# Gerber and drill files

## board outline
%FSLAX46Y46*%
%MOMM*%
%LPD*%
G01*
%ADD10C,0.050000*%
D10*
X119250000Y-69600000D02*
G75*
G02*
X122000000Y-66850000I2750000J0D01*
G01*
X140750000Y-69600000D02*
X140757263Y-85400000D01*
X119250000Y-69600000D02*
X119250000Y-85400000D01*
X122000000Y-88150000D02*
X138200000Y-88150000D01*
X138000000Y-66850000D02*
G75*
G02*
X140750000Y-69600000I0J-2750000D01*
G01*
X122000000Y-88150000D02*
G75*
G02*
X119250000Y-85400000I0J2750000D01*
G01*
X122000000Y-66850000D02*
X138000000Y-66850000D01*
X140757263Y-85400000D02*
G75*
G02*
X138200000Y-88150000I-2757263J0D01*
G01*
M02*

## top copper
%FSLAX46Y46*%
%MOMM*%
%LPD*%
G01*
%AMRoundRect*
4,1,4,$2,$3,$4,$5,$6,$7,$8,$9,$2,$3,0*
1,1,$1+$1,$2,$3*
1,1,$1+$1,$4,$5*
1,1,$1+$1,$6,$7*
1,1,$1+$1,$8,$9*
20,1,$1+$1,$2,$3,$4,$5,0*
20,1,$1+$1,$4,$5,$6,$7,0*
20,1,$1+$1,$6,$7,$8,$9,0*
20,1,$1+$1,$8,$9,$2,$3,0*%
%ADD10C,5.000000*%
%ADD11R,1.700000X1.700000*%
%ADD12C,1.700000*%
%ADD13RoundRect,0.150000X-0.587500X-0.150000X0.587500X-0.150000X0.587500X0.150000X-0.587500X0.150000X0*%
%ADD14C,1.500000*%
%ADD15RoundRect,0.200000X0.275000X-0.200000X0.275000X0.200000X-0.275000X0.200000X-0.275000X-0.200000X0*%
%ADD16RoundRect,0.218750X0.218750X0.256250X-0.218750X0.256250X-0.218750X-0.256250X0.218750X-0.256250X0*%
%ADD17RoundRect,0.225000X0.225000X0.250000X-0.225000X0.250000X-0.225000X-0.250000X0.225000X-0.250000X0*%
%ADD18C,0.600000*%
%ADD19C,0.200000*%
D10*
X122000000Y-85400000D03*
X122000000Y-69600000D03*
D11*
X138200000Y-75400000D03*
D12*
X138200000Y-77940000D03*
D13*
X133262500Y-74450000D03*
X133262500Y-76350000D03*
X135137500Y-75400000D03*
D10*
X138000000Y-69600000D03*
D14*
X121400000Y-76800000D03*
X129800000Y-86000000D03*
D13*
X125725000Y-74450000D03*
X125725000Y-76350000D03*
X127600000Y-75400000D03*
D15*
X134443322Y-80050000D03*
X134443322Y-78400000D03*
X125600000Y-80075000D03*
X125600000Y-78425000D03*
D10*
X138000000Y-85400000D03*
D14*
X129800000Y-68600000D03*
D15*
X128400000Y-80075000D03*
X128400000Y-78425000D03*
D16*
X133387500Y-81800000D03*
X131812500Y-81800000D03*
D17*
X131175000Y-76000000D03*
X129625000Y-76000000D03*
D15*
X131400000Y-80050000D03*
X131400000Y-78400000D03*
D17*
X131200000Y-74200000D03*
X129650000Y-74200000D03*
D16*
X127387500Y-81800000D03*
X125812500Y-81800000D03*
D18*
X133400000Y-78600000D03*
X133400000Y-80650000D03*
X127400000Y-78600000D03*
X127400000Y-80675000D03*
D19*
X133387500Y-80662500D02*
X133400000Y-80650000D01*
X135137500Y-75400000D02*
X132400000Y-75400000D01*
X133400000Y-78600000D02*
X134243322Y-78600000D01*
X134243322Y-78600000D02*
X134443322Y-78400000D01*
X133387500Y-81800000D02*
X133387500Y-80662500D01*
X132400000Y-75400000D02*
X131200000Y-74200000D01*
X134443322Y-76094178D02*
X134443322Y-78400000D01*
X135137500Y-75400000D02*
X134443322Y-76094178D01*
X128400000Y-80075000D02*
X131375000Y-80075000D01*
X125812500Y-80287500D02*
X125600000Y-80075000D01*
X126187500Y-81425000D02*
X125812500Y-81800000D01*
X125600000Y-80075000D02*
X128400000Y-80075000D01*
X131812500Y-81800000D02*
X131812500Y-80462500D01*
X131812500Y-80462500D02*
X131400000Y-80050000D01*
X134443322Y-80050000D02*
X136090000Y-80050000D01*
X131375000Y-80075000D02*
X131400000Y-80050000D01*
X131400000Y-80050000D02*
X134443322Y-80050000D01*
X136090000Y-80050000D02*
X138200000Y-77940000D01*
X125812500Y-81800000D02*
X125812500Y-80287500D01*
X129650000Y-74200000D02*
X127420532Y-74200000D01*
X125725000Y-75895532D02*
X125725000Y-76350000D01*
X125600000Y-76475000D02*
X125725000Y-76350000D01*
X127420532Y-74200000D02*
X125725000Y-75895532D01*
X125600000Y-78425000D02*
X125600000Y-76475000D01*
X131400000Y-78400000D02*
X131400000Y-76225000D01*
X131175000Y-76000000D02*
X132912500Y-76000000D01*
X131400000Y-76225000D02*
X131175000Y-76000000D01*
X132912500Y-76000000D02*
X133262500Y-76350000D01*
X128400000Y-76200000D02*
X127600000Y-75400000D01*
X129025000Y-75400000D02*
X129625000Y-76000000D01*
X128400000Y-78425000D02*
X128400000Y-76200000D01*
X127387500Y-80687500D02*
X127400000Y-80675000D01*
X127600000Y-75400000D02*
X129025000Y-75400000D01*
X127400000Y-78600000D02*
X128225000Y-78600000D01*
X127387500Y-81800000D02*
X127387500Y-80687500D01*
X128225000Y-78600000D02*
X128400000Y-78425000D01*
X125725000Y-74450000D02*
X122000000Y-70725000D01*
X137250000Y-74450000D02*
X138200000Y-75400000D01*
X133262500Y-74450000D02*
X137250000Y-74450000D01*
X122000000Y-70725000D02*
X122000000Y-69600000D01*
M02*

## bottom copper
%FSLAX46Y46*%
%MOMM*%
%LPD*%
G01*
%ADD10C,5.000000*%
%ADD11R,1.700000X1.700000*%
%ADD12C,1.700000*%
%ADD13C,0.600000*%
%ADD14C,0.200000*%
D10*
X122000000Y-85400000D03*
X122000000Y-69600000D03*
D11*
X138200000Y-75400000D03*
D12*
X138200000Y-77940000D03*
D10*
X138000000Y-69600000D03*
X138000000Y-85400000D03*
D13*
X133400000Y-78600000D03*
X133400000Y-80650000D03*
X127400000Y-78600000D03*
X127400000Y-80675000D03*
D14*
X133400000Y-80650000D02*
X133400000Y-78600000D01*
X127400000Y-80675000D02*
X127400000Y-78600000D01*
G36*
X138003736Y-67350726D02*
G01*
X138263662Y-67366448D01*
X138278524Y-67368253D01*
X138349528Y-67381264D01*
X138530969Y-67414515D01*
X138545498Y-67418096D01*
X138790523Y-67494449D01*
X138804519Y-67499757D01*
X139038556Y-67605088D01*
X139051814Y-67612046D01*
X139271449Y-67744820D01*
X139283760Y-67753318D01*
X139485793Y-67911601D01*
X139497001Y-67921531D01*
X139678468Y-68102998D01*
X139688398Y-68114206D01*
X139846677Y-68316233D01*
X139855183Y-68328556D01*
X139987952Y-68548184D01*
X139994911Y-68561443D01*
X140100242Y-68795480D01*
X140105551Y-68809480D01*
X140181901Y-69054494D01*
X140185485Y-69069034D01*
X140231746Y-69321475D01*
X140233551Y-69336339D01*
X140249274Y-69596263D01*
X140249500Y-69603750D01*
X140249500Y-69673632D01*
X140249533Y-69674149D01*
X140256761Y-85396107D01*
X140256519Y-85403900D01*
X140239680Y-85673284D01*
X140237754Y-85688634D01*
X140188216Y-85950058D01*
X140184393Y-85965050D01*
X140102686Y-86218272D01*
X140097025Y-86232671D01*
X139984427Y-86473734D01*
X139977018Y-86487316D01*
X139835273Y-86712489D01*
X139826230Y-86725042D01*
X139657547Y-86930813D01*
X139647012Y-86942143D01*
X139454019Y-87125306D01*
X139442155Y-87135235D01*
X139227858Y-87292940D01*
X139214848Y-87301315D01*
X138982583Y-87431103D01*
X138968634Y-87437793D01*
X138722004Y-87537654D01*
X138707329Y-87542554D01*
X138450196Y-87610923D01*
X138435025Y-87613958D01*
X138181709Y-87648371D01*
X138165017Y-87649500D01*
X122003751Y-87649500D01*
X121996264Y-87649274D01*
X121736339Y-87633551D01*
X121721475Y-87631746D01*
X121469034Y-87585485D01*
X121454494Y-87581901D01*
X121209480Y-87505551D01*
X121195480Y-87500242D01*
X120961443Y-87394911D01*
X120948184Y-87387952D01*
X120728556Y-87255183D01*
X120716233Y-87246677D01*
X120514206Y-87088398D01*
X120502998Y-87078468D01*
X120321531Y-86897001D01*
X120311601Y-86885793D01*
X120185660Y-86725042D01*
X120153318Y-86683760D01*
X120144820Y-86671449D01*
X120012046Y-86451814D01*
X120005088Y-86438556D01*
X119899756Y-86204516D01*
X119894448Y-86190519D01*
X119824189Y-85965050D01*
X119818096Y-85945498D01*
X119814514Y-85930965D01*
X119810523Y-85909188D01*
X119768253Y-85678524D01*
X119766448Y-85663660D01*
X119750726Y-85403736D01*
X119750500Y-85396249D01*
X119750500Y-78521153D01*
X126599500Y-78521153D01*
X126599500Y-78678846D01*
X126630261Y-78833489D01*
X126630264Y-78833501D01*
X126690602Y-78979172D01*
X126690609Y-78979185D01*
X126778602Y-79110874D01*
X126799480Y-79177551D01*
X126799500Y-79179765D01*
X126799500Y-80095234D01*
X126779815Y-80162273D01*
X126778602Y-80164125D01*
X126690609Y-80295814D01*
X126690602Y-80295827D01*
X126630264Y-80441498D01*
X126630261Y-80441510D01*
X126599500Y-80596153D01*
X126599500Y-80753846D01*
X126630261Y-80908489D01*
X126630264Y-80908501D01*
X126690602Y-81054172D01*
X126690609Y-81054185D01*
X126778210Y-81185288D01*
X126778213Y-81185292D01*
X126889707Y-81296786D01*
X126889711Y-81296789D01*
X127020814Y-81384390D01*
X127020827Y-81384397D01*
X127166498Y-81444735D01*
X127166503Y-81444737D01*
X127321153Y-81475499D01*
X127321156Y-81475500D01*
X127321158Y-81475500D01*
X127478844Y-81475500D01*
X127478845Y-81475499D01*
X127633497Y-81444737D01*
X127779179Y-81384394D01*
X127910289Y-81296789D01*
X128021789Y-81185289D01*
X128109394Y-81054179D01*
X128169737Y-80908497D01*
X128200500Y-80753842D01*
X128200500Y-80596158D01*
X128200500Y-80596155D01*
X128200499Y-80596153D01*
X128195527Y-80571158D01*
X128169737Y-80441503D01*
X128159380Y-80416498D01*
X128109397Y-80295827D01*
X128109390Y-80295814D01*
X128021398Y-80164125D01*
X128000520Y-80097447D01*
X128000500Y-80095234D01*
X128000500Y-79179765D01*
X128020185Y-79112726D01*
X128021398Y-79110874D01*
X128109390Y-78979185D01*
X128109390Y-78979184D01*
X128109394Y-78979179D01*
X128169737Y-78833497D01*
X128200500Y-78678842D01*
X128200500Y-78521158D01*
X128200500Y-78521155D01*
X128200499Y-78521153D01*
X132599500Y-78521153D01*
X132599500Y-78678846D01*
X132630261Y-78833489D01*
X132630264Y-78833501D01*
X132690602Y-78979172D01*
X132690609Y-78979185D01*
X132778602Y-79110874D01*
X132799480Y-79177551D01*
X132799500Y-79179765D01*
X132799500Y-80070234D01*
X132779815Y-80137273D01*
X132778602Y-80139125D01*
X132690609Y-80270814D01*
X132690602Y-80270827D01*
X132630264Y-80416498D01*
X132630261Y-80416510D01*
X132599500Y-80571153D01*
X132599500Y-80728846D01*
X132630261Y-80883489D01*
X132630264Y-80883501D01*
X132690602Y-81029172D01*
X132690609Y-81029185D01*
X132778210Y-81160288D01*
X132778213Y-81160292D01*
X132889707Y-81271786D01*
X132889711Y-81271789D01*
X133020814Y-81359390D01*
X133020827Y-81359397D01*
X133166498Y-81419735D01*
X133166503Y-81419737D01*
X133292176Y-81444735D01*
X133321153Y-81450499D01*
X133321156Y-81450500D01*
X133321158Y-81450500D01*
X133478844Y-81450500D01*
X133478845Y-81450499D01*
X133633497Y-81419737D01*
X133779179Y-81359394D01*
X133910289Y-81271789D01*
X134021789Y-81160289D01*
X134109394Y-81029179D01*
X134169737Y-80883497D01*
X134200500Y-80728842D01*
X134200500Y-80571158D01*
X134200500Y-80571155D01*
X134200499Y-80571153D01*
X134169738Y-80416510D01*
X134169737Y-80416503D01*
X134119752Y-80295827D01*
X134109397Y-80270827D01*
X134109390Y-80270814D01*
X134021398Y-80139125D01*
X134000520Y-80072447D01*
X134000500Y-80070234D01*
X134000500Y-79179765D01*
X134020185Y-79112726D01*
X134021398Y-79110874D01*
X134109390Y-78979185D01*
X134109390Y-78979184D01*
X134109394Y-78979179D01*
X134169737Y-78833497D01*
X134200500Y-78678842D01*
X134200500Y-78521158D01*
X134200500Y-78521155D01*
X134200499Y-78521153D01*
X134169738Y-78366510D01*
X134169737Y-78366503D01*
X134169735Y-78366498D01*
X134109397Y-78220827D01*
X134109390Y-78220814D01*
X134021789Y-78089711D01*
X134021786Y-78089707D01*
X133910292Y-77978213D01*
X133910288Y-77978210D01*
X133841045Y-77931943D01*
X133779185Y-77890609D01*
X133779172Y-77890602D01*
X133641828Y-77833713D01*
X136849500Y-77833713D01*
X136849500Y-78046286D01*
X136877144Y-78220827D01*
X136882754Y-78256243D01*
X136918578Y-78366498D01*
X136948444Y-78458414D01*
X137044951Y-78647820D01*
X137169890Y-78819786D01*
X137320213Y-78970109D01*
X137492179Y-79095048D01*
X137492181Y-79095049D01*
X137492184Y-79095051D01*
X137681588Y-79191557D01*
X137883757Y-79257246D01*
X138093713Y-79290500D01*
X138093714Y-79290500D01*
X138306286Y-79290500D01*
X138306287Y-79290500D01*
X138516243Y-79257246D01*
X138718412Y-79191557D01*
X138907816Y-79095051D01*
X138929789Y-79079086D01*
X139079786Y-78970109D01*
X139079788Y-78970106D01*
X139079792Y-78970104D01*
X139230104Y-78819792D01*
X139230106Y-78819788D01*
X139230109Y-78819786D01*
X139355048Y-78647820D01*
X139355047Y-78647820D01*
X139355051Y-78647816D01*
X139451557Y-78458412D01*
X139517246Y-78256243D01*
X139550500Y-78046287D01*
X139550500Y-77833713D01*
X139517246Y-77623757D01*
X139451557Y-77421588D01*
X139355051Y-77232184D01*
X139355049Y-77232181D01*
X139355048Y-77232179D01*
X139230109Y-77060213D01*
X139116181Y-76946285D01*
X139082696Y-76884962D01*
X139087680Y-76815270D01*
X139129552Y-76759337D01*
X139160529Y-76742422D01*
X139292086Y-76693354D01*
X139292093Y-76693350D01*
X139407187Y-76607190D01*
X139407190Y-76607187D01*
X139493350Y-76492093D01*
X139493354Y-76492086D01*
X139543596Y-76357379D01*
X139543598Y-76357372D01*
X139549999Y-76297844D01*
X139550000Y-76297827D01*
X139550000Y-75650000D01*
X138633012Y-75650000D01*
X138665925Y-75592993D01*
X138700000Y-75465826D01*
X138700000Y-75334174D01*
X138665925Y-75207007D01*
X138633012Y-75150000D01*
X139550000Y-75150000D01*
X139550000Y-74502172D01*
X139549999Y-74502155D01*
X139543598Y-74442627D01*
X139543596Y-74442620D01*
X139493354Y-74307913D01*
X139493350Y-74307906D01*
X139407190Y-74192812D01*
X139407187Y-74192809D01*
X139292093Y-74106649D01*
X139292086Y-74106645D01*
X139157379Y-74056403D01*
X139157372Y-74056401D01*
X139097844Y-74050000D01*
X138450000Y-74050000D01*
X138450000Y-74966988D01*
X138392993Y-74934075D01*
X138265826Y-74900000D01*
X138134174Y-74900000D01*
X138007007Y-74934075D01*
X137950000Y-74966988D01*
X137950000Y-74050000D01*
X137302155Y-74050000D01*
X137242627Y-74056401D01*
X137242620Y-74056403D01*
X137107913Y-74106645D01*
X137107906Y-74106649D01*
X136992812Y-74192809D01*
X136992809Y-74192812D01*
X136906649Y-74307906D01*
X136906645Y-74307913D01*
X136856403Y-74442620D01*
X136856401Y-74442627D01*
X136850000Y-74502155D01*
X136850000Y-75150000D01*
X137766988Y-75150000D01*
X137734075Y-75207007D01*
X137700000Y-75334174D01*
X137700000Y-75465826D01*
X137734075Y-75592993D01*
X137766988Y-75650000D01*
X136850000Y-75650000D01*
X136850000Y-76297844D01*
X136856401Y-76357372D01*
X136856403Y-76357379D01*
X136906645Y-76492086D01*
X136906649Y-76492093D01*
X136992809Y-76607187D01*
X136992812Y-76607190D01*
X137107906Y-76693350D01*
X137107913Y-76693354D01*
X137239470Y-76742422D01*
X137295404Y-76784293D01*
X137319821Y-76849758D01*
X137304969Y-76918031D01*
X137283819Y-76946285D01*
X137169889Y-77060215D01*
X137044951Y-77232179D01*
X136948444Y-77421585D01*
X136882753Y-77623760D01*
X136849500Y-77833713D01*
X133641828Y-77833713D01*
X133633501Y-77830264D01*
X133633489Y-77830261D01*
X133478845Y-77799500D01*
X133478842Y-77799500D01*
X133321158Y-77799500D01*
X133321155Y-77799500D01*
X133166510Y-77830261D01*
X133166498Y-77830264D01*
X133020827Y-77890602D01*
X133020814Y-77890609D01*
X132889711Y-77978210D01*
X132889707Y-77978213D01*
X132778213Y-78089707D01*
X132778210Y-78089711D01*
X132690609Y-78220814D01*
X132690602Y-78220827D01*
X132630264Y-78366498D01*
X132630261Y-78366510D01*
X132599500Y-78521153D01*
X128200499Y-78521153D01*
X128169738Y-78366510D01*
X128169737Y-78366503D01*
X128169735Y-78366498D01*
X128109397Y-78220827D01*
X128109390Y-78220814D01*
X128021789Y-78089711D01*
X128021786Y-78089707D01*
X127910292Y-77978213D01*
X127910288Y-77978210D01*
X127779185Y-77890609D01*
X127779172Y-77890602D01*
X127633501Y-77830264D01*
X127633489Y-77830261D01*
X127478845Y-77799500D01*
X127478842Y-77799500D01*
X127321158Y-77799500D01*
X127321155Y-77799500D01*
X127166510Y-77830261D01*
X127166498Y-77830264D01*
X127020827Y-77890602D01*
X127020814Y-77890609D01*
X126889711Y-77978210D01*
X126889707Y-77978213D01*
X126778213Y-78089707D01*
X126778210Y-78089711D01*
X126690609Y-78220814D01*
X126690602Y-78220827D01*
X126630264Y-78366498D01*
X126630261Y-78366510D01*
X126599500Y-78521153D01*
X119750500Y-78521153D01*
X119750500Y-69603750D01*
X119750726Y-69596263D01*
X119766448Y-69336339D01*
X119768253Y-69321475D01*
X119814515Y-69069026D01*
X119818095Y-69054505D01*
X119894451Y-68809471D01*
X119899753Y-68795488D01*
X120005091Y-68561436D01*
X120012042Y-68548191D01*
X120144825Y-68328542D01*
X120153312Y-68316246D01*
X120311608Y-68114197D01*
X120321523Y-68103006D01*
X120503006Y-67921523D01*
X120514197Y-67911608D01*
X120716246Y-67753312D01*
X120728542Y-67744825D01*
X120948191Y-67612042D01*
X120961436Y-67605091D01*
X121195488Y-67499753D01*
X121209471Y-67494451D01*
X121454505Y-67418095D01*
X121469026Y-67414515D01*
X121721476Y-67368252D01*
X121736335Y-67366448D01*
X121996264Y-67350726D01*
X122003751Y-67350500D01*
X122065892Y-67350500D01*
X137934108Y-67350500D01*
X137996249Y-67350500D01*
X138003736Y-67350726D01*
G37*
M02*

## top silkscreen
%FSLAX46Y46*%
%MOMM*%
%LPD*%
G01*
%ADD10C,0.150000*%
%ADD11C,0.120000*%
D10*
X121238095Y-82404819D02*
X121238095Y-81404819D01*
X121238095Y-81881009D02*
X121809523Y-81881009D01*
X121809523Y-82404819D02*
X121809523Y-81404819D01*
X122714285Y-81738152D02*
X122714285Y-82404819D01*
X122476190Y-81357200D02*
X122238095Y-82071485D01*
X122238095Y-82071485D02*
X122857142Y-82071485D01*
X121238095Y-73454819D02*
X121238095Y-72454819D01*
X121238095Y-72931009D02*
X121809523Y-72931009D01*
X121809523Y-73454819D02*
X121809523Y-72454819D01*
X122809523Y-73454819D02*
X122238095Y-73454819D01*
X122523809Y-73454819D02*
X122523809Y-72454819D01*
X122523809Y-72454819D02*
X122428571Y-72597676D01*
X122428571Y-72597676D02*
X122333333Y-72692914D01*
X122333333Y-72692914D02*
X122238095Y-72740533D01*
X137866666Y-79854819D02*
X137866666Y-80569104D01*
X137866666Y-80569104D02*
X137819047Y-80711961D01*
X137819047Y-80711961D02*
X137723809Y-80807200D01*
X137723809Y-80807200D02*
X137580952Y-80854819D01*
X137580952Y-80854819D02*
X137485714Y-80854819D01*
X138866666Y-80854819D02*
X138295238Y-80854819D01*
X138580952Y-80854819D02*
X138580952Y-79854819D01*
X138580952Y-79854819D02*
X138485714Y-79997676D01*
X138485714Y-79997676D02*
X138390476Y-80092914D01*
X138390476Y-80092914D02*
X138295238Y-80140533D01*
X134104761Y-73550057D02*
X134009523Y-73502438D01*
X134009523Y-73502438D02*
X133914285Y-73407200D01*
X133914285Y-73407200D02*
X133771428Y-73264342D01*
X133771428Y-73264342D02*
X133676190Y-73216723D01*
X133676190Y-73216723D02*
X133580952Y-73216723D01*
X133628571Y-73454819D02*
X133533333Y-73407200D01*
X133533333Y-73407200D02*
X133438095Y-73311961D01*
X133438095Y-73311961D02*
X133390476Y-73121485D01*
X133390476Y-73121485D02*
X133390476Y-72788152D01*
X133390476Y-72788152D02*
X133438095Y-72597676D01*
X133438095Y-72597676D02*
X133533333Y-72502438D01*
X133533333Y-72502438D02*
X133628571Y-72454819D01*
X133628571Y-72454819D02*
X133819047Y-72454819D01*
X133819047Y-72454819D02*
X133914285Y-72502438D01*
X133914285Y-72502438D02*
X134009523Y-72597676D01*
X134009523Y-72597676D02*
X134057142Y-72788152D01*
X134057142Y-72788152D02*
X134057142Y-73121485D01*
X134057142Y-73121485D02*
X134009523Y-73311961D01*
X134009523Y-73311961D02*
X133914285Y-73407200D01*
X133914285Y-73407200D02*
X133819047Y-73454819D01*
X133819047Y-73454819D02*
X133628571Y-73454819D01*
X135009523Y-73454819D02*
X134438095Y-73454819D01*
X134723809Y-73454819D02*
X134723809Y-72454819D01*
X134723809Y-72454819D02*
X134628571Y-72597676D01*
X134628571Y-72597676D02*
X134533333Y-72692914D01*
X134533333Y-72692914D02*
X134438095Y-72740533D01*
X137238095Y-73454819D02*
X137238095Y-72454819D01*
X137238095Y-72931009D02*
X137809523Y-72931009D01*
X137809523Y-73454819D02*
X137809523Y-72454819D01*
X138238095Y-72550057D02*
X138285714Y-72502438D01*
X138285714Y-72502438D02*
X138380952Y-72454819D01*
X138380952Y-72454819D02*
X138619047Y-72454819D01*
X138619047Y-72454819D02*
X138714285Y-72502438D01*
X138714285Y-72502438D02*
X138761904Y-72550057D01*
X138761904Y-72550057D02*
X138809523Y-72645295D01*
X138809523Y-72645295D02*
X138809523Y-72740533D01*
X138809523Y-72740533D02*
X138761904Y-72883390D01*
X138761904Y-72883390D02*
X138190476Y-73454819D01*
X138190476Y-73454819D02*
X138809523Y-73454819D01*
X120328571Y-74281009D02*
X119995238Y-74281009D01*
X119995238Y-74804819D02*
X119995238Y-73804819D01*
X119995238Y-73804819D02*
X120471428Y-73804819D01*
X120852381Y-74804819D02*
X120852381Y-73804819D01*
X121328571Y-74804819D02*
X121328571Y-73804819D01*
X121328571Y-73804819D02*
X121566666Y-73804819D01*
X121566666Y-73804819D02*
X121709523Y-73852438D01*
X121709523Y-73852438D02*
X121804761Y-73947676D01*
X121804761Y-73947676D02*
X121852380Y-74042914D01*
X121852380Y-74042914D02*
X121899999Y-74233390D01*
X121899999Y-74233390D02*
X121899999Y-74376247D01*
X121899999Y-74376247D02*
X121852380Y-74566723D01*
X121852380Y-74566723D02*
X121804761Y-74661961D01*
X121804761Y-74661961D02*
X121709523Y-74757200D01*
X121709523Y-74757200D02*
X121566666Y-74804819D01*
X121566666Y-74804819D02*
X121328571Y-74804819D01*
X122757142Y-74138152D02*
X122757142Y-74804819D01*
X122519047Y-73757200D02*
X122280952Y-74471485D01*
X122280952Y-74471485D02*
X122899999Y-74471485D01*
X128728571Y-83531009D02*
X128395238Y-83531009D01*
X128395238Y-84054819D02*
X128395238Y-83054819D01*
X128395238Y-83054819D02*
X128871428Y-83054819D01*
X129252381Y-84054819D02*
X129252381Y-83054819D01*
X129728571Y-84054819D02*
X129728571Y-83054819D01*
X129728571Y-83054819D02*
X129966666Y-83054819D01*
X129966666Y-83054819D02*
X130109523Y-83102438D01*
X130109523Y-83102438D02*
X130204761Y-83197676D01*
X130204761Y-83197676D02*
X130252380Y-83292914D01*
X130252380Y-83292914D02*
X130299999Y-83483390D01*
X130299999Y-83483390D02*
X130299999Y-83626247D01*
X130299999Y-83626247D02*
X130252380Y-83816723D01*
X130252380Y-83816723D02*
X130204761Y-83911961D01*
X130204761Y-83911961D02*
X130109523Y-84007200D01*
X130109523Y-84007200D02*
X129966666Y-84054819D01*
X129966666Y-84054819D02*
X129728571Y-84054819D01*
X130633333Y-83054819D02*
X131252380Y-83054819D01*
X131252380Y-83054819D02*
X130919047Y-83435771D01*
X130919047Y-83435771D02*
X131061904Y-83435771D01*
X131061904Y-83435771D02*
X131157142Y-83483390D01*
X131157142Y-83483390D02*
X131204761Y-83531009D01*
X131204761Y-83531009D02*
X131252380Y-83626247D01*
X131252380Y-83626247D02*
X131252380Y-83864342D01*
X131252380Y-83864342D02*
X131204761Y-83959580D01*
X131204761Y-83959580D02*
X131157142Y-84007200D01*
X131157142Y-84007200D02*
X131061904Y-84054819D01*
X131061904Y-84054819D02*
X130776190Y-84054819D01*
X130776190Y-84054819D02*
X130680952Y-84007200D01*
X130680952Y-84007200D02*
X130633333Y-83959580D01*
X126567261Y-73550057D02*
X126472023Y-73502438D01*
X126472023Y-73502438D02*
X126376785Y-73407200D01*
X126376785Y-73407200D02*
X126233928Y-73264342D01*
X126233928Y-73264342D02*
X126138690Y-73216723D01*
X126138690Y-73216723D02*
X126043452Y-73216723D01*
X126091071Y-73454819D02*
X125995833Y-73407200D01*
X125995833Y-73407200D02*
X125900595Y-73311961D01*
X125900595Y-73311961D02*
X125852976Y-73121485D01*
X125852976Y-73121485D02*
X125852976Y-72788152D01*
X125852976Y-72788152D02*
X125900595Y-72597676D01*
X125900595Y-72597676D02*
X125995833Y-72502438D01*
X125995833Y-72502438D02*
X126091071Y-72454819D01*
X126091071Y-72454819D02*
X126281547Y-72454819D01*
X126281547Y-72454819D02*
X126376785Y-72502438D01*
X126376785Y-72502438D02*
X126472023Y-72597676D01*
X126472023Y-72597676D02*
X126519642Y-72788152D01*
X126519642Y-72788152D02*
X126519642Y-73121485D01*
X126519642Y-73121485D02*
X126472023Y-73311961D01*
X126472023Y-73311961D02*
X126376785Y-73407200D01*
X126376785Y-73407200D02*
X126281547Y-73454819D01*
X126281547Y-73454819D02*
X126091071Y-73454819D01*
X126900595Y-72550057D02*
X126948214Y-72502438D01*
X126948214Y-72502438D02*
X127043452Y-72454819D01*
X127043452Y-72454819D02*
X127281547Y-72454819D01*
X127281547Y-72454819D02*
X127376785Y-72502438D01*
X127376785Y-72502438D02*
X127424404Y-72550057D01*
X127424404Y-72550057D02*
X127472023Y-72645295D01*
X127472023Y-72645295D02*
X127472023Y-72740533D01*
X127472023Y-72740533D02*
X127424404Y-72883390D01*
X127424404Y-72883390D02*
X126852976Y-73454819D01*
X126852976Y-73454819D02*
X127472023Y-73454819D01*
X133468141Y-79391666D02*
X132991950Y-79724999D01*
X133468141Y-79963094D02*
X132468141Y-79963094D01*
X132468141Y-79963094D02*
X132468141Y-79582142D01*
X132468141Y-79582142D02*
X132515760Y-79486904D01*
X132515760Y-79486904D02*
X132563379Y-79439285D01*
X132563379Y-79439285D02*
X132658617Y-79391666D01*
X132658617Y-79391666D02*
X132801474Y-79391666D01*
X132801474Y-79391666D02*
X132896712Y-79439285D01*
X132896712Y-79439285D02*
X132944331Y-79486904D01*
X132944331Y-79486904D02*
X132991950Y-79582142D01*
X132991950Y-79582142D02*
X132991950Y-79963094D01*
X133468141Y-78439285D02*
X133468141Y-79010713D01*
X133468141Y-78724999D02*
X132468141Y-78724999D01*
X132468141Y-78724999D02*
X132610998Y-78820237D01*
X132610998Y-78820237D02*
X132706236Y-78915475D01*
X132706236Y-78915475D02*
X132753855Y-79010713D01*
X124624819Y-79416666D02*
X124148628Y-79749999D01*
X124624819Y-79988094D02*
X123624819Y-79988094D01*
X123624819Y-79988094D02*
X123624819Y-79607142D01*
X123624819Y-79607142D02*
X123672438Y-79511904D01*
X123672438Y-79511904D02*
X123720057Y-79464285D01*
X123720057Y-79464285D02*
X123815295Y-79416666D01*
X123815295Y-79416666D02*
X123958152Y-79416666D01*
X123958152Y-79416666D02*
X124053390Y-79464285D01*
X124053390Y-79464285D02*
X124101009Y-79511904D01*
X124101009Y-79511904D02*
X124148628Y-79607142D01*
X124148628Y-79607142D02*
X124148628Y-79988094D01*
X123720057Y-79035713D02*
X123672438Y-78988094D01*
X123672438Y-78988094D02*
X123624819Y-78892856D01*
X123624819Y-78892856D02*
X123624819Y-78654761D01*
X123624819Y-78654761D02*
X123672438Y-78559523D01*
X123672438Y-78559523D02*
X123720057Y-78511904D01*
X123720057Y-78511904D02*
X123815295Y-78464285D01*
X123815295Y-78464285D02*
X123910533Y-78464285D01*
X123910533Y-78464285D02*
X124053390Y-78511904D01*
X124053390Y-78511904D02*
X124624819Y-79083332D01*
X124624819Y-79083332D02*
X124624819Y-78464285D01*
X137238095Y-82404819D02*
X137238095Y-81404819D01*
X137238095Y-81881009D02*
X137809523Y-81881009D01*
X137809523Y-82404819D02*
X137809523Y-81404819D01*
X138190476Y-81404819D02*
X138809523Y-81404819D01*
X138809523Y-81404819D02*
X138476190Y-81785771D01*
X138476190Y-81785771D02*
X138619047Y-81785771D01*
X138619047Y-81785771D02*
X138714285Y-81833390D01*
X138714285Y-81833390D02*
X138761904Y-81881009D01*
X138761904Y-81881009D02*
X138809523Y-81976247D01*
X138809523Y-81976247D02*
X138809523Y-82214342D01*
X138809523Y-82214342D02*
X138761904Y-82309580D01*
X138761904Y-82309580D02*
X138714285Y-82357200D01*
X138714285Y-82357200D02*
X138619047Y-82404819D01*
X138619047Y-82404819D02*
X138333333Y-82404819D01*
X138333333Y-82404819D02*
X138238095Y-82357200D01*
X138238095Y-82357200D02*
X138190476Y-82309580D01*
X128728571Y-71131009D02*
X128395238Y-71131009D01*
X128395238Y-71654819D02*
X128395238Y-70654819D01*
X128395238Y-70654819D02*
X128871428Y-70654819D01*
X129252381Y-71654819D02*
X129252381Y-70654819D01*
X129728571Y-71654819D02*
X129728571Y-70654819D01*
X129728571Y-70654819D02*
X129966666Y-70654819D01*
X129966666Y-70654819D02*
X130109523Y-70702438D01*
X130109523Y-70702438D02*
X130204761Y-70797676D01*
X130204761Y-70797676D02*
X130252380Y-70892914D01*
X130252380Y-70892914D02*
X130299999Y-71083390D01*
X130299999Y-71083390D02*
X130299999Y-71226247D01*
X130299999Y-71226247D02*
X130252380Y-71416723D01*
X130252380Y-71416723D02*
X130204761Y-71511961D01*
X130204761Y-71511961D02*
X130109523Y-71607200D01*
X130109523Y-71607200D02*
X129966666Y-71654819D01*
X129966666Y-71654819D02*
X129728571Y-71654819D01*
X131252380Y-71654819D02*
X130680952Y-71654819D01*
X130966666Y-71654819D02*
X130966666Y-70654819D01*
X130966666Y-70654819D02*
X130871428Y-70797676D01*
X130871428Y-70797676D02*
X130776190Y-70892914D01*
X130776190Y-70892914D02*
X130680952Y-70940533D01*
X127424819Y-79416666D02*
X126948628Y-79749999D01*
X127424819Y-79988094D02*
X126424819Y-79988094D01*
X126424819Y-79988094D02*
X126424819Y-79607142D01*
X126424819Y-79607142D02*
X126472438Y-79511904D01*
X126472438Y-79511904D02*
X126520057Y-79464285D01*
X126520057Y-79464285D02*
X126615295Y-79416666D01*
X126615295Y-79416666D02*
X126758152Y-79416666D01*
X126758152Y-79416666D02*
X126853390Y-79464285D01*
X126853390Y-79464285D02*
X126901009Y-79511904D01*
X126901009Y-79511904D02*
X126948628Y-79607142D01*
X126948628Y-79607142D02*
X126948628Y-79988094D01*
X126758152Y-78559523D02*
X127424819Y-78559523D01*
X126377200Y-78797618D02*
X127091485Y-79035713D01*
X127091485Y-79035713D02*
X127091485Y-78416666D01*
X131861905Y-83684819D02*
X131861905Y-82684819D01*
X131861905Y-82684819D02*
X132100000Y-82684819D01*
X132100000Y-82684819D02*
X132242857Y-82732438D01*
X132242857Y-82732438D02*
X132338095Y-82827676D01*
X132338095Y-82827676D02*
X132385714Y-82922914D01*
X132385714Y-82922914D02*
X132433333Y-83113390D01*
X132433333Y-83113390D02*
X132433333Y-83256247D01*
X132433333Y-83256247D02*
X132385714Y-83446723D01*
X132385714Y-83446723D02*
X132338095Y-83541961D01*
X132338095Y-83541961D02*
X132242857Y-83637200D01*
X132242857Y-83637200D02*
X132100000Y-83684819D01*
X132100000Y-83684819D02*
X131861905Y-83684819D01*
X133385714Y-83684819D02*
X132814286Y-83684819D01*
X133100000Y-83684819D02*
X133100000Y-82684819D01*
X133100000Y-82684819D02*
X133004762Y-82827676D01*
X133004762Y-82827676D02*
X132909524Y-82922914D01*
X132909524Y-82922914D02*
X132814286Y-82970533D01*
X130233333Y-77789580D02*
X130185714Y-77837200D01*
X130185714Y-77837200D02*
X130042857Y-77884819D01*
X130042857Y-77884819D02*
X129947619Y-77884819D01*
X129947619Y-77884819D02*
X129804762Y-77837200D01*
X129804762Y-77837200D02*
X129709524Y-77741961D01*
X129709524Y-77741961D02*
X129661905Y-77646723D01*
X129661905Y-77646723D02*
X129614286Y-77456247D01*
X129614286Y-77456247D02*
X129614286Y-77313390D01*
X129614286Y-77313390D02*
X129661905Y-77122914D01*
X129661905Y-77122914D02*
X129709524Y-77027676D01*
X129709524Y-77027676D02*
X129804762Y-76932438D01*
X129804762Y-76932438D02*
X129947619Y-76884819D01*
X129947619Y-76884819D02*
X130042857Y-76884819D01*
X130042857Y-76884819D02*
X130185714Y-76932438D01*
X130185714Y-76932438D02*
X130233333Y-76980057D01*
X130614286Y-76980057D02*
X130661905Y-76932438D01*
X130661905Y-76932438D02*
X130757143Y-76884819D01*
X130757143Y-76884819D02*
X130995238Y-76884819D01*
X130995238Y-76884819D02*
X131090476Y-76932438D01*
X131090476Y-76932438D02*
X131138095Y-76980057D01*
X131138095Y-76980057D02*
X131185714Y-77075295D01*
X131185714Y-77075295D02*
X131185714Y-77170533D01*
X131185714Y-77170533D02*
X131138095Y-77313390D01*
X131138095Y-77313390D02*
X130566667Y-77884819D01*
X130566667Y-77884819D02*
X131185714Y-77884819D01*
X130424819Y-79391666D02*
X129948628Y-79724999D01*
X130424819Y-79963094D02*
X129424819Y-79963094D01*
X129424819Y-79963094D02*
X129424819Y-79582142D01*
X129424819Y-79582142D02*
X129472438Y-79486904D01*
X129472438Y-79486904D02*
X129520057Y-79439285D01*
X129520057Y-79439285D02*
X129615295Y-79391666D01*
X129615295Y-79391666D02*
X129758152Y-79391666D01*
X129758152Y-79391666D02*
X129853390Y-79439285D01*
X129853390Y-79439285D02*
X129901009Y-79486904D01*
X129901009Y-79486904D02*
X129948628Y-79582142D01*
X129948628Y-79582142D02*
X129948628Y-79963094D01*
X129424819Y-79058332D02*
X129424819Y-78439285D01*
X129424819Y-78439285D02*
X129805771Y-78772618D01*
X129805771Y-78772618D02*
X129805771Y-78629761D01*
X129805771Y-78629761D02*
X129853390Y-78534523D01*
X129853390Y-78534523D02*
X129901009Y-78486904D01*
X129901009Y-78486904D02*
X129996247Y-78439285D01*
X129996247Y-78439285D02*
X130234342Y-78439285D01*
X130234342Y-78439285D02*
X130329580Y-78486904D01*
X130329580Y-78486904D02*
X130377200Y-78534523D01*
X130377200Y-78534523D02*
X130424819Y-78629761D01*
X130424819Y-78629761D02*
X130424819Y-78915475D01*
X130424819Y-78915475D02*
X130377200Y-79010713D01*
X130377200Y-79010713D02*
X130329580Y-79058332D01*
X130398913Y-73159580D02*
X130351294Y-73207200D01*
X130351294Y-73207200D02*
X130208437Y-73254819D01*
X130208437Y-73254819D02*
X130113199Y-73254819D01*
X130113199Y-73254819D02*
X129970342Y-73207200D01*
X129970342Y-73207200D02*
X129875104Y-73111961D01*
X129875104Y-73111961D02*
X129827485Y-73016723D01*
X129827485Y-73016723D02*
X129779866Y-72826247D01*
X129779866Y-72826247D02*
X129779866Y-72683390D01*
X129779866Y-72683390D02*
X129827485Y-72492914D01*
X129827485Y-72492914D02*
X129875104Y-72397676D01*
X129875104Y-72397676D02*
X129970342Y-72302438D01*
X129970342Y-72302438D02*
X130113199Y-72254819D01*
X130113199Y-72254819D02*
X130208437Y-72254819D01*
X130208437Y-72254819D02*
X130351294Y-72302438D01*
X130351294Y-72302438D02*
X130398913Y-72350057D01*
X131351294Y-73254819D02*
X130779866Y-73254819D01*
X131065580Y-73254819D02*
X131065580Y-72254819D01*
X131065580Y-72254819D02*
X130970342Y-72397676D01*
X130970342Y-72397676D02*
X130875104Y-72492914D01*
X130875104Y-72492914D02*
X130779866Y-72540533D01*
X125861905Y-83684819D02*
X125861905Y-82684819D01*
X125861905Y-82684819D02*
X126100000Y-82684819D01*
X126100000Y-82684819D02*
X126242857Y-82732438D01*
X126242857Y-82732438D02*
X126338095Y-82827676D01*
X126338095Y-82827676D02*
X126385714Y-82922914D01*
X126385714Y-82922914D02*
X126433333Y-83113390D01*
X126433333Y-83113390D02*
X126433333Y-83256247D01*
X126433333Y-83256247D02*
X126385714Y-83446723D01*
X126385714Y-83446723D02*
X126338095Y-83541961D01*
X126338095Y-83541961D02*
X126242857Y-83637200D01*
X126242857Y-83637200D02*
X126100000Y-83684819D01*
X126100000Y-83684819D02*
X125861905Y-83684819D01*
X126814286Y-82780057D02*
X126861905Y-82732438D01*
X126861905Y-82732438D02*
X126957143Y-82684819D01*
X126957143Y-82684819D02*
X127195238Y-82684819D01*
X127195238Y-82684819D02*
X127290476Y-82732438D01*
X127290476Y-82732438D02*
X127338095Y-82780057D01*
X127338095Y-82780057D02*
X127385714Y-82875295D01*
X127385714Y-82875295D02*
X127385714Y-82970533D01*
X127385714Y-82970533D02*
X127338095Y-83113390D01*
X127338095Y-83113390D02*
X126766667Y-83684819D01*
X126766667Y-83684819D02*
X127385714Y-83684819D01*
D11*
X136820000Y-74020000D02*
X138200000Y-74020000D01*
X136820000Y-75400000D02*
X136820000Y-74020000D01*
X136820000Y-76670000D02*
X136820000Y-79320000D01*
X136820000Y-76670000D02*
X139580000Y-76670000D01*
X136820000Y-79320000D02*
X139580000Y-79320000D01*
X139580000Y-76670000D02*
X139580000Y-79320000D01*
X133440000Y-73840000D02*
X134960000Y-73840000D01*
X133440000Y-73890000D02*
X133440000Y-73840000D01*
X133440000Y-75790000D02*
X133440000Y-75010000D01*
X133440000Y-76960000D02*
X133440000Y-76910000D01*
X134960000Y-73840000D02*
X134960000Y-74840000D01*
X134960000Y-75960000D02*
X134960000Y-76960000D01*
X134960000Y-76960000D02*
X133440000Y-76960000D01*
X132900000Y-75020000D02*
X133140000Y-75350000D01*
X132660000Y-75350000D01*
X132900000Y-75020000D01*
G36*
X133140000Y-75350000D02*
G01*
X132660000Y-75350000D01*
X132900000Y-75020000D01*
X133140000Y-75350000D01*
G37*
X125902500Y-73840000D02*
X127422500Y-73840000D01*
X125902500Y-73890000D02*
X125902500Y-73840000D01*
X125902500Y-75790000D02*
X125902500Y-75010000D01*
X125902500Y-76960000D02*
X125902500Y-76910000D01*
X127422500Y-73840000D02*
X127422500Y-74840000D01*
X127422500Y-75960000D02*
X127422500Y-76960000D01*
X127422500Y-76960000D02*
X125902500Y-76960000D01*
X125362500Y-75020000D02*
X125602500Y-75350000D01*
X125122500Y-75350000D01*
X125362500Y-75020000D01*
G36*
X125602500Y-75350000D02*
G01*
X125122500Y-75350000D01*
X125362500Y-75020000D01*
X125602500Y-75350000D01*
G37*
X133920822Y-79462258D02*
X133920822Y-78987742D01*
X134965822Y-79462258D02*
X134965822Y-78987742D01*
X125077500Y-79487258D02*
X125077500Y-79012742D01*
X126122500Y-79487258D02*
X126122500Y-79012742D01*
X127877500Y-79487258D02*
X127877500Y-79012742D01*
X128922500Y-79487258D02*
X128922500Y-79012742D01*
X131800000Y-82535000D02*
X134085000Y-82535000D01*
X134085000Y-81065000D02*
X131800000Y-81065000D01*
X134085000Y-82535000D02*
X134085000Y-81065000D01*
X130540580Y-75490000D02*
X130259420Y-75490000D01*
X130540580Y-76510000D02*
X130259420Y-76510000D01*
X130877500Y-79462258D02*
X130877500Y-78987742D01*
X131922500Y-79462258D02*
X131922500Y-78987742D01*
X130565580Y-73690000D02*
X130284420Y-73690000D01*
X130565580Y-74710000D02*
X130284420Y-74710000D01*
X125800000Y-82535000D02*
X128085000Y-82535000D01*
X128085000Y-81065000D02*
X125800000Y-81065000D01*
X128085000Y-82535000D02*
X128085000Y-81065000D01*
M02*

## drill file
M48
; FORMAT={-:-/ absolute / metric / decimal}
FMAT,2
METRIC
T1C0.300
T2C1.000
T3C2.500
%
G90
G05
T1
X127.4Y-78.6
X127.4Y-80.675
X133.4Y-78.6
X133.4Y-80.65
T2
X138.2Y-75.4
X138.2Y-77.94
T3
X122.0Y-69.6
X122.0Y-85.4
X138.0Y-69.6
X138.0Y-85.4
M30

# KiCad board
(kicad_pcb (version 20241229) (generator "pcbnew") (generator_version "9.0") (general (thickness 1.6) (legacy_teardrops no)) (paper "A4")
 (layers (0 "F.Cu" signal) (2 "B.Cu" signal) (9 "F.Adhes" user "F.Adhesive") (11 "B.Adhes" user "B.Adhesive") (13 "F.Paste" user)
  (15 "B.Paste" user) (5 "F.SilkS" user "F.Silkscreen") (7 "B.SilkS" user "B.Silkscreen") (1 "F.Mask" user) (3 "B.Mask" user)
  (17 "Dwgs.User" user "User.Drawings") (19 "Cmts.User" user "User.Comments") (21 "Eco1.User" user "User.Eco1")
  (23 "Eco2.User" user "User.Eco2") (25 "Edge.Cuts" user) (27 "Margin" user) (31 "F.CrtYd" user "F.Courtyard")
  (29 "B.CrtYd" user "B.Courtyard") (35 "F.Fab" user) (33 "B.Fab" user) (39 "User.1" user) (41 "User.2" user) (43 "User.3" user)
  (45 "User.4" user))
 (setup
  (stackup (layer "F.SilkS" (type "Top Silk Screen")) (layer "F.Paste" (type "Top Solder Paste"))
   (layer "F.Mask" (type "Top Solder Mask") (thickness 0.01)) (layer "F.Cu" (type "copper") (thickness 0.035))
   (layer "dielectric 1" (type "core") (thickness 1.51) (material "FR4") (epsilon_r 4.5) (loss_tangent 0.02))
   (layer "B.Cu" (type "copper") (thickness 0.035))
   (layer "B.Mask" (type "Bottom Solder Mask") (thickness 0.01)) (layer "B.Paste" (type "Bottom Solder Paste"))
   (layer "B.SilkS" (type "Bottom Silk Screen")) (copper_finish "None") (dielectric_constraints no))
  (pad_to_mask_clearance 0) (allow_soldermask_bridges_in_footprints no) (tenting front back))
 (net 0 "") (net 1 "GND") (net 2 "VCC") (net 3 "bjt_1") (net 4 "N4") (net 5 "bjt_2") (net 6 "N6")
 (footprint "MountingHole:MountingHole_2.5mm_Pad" (layer "F.Cu") (at 122 85.4)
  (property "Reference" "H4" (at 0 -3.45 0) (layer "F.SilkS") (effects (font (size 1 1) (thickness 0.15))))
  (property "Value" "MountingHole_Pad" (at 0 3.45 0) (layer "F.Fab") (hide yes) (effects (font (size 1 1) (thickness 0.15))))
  (pad "1" thru_hole circle (at 0 0) (size 5 5) (drill 2.5) (layers "*.Cu" "*.Mask") (remove_unused_layers no) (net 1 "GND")
   (zone_connect 2)))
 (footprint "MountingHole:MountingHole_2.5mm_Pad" (layer "F.Cu") (at 122 69.6)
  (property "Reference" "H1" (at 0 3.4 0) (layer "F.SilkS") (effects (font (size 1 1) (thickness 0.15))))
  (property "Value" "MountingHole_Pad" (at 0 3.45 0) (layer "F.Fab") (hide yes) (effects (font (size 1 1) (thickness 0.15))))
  (pad "1" thru_hole circle (at 0 0) (size 5 5) (drill 2.5) (layers "*.Cu" "*.Mask") (remove_unused_layers no) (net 1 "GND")
   (zone_connect 2)))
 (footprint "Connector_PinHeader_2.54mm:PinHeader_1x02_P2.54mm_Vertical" (layer "F.Cu") (at 138.2 75.4)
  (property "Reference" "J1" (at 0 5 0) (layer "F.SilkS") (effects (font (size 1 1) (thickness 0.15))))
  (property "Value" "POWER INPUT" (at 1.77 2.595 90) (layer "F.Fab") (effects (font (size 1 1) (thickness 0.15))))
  (fp_line (start -1.38 -1.38) (end 0 -1.38) (stroke (width 0.12) (type solid)) (layer "F.SilkS"))
  (fp_line (start -1.38 0) (end -1.38 -1.38) (stroke (width 0.12) (type solid)) (layer "F.SilkS"))
  (fp_line (start -1.38 1.27) (end -1.38 3.92) (stroke (width 0.12) (type solid)) (layer "F.SilkS"))
  (fp_line (start -1.38 1.27) (end 1.38 1.27) (stroke (width 0.12) (type solid)) (layer "F.SilkS"))
  (fp_line (start -1.38 3.92) (end 1.38 3.92) (stroke (width 0.12) (type solid)) (layer "F.SilkS"))
  (fp_line (start 1.38 1.27) (end 1.38 3.92) (stroke (width 0.12) (type solid)) (layer "F.SilkS"))
  (pad "1" thru_hole rect (at 0 0) (size 1.7 1.7) (drill 1) (layers "*.Cu" "*.Mask") (remove_unused_layers no) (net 1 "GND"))
  (pad "2" thru_hole circle (at 0 2.54) (size 1.7 1.7) (drill 1) (layers "*.Cu" "*.Mask") (remove_unused_layers no) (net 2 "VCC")))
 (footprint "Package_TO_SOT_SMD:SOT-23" (layer "F.Cu") (at 134.2 75.4)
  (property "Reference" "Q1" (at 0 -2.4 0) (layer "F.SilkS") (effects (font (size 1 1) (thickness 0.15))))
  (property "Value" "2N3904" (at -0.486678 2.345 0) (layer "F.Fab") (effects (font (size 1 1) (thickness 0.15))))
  (fp_line (start -0.76 -1.56) (end 0.76 -1.56) (stroke (width 0.12) (type solid)) (layer "F.SilkS"))
  (fp_line (start -0.76 -1.51) (end -0.76 -1.56) (stroke (width 0.12) (type solid)) (layer "F.SilkS"))
  (fp_line (start -0.76 0.39) (end -0.76 -0.39) (stroke (width 0.12) (type solid)) (layer "F.SilkS"))
  (fp_line (start -0.76 1.56) (end -0.76 1.51) (stroke (width 0.12) (type solid)) (layer "F.SilkS"))
  (fp_line (start 0.76 -1.56) (end 0.76 -0.56) (stroke (width 0.12) (type solid)) (layer "F.SilkS"))
  (fp_line (start 0.76 0.56) (end 0.76 1.56) (stroke (width 0.12) (type solid)) (layer "F.SilkS"))
  (fp_line (start 0.76 1.56) (end -0.76 1.56) (stroke (width 0.12) (type solid)) (layer "F.SilkS"))
  (fp_poly (pts (xy -1.3 -0.38) (xy -1.06 -0.05) (xy -1.54 -0.05)) (stroke (width 0.12) (type solid)) (fill yes) (layer "F.SilkS"))
  (pad "1" smd roundrect (at -0.9375 -0.95) (size 1.475 0.6) (layers "F.Cu" "F.Mask" "F.Paste") (roundrect_rratio 0.25) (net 1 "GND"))
  (pad "2" smd roundrect (at -0.9375 0.95) (size 1.475 0.6) (layers "F.Cu" "F.Mask" "F.Paste") (roundrect_rratio 0.25) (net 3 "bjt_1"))
  (pad "3" smd roundrect (at 0.9375 0) (size 1.475 0.6) (layers "F.Cu" "F.Mask" "F.Paste") (roundrect_rratio 0.25) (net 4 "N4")))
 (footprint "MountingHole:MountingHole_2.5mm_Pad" (layer "F.Cu") (at 138 69.6)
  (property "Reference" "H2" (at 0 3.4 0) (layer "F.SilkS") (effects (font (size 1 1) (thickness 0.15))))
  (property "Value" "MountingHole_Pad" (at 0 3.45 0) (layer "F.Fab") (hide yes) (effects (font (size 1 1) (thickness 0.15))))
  (pad "1" thru_hole circle (at 0 0) (size 5 5) (drill 2.5) (layers "*.Cu" "*.Mask") (remove_unused_layers no) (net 1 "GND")
   (zone_connect 2)))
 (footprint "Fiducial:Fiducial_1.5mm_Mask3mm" (layer "F.Cu") (at 121.4 76.8)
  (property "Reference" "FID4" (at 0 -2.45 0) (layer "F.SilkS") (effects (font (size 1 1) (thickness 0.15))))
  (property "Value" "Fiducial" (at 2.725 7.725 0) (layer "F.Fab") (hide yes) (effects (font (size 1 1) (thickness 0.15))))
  (pad "" smd circle (at 0 0) (size 1.5 1.5) (layers "F.Cu" "F.Mask") (solder_mask_margin 0.75) (clearance 0.85)))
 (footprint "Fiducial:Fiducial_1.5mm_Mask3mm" (layer "F.Cu") (at 129.8 86)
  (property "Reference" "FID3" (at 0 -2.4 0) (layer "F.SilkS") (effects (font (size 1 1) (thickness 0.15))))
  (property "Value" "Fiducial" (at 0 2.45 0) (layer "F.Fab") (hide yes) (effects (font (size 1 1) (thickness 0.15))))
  (pad "" smd circle (at 0 0) (size 1.5 1.5) (layers "F.Cu" "F.Mask") (solder_mask_margin 0.75) (clearance 0.85)))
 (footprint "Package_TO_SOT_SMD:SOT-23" (layer "F.Cu") (at 126.6625 75.4)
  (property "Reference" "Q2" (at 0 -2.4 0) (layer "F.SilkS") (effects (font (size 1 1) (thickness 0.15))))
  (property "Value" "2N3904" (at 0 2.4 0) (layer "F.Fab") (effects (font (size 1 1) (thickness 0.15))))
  (fp_line (start -0.76 -1.56) (end 0.76 -1.56) (stroke (width 0.12) (type solid)) (layer "F.SilkS"))
  (fp_line (start -0.76 -1.51) (end -0.76 -1.56) (stroke (width 0.12) (type solid)) (layer "F.SilkS"))
  (fp_line (start -0.76 0.39) (end -0.76 -0.39) (stroke (width 0.12) (type solid)) (layer "F.SilkS"))
  (fp_line (start -0.76 1.56) (end -0.76 1.51) (stroke (width 0.12) (type solid)) (layer "F.SilkS"))
  (fp_line (start 0.76 -1.56) (end 0.76 -0.56) (stroke (width 0.12) (type solid)) (layer "F.SilkS"))
  (fp_line (start 0.76 0.56) (end 0.76 1.56) (stroke (width 0.12) (type solid)) (layer "F.SilkS"))
  (fp_line (start 0.76 1.56) (end -0.76 1.56) (stroke (width 0.12) (type solid)) (layer "F.SilkS"))
  (fp_poly (pts (xy -1.3 -0.38) (xy -1.06 -0.05) (xy -1.54 -0.05)) (stroke (width 0.12) (type solid)) (fill yes) (layer "F.SilkS"))
  (pad "1" smd roundrect (at -0.9375 -0.95) (size 1.475 0.6) (layers "F.Cu" "F.Mask" "F.Paste") (roundrect_rratio 0.25) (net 1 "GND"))
  (pad "2" smd roundrect (at -0.9375 0.95) (size 1.475 0.6) (layers "F.Cu" "F.Mask" "F.Paste") (roundrect_rratio 0.25) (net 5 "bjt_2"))
  (pad "3" smd roundrect (at 0.9375 0) (size 1.475 0.6) (layers "F.Cu" "F.Mask" "F.Paste") (roundrect_rratio 0.25) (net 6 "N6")))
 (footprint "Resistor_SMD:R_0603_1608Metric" (layer "F.Cu") (at 134.443322 79.225 90)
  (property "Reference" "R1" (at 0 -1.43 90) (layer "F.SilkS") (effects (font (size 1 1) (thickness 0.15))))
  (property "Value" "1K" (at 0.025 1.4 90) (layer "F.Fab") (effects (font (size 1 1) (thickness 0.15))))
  (fp_line (start -0.237258 -0.5225) (end 0.237258 -0.5225) (stroke (width 0.12) (type solid)) (layer "F.SilkS"))
  (fp_line (start -0.237258 0.5225) (end 0.237258 0.5225) (stroke (width 0.12) (type solid)) (layer "F.SilkS"))
  (pad "1" smd roundrect (at -0.825 0 90) (size 0.8 0.95) (layers "F.Cu" "F.Mask" "F.Paste") (roundrect_rratio 0.25) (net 2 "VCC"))
  (pad "2" smd roundrect (at 0.825 0 90) (size 0.8 0.95) (layers "F.Cu" "F.Mask" "F.Paste") (roundrect_rratio 0.25) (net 4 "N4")))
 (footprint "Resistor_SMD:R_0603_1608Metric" (layer "F.Cu") (at 125.6 79.25 90)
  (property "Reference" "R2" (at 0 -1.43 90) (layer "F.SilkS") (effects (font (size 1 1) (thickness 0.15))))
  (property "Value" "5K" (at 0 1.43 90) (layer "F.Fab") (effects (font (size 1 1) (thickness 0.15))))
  (fp_line (start -0.237258 -0.5225) (end 0.237258 -0.5225) (stroke (width 0.12) (type solid)) (layer "F.SilkS"))
  (fp_line (start -0.237258 0.5225) (end 0.237258 0.5225) (stroke (width 0.12) (type solid)) (layer "F.SilkS"))
  (pad "1" smd roundrect (at -0.825 0 90) (size 0.8 0.95) (layers "F.Cu" "F.Mask" "F.Paste") (roundrect_rratio 0.25) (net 2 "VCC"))
  (pad "2" smd roundrect (at 0.825 0 90) (size 0.8 0.95) (layers "F.Cu" "F.Mask" "F.Paste") (roundrect_rratio 0.25) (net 5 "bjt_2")))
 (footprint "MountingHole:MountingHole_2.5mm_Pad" (layer "F.Cu") (at 138 85.4)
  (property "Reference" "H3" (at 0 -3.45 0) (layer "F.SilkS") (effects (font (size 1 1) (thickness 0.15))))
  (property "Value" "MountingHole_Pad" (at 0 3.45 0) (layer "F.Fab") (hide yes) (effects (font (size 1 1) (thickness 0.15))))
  (pad "1" thru_hole circle (at 0 0) (size 5 5) (drill 2.5) (layers "*.Cu" "*.Mask") (remove_unused_layers no) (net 1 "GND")
   (zone_connect 2)))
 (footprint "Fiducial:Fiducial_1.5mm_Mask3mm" (layer "F.Cu") (at 129.8 68.6)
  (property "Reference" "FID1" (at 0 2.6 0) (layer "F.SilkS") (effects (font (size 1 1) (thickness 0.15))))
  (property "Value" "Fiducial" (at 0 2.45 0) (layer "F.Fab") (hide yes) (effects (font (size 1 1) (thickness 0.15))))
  (pad "" smd circle (at 0 0) (size 1.5 1.5) (layers "F.Cu" "F.Mask") (solder_mask_margin 0.75) (clearance 0.85)))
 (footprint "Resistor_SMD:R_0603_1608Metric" (layer "F.Cu") (at 128.4 79.25 90)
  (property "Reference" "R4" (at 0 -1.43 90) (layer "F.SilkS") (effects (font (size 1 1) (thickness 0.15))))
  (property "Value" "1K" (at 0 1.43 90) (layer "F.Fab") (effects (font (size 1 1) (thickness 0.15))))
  (fp_line (start -0.237258 -0.5225) (end 0.237258 -0.5225) (stroke (width 0.12) (type solid)) (layer "F.SilkS"))
  (fp_line (start -0.237258 0.5225) (end 0.237258 0.5225) (stroke (width 0.12) (type solid)) (layer "F.SilkS"))
  (pad "1" smd roundrect (at -0.825 0 90) (size 0.8 0.95) (layers "F.Cu" "F.Mask" "F.Paste") (roundrect_rratio 0.25) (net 2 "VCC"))
  (pad "2" smd roundrect (at 0.825 0 90) (size 0.8 0.95) (layers "F.Cu" "F.Mask" "F.Paste") (roundrect_rratio 0.25) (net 6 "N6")))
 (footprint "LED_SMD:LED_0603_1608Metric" (layer "F.Cu") (at 132.6 81.8 180)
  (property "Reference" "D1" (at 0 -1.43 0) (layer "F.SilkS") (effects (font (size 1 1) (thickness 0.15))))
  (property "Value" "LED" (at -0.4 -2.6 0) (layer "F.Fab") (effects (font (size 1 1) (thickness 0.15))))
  (fp_line (start 0.8 -0.735) (end -1.485 -0.735) (stroke (width 0.12) (type solid)) (layer "F.SilkS"))
  (fp_line (start -1.485 0.735) (end 0.8 0.735) (stroke (width 0.12) (type solid)) (layer "F.SilkS"))
  (fp_line (start -1.485 -0.735) (end -1.485 0.735) (stroke (width 0.12) (type solid)) (layer "F.SilkS"))
  (pad "1" smd roundrect (at -0.7875 0 180) (size 0.875 0.95) (layers "F.Cu" "F.Mask" "F.Paste") (roundrect_rratio 0.25) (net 4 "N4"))
  (pad "2" smd roundrect (at 0.7875 0 180) (size 0.875 0.95) (layers "F.Cu" "F.Mask" "F.Paste") (roundrect_rratio 0.25) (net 2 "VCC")))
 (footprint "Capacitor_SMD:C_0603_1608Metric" (layer "F.Cu") (at 130.4 76 180)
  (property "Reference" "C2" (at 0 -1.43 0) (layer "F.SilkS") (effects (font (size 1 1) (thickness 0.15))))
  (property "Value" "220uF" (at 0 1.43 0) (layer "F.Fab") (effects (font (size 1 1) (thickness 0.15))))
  (fp_line (start -0.14058 0.51) (end 0.14058 0.51) (stroke (width 0.12) (type solid)) (layer "F.SilkS"))
  (fp_line (start -0.14058 -0.51) (end 0.14058 -0.51) (stroke (width 0.12) (type solid)) (layer "F.SilkS"))
  (pad "1" smd roundrect (at -0.775 0 180) (size 0.9 0.95) (layers "F.Cu" "F.Mask" "F.Paste") (roundrect_rratio 0.25) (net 3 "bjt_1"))
  (pad "2" smd roundrect (at 0.775 0 180) (size 0.9 0.95) (layers "F.Cu" "F.Mask" "F.Paste") (roundrect_rratio 0.25) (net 6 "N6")))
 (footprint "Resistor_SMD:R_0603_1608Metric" (layer "F.Cu") (at 131.4 79.225 90)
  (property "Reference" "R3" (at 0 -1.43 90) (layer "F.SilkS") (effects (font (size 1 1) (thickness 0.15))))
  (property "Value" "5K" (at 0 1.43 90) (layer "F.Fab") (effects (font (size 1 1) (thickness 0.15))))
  (fp_line (start -0.237258 -0.5225) (end 0.237258 -0.5225) (stroke (width 0.12) (type solid)) (layer "F.SilkS"))
  (fp_line (start -0.237258 0.5225) (end 0.237258 0.5225) (stroke (width 0.12) (type solid)) (layer "F.SilkS"))
  (pad "1" smd roundrect (at -0.825 0 90) (size 0.8 0.95) (layers "F.Cu" "F.Mask" "F.Paste") (roundrect_rratio 0.25) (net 2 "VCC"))
  (pad "2" smd roundrect (at 0.825 0 90) (size 0.8 0.95) (layers "F.Cu" "F.Mask" "F.Paste") (roundrect_rratio 0.25) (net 3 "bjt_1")))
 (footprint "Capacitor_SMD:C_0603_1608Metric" (layer "F.Cu") (at 130.425 74.2 180)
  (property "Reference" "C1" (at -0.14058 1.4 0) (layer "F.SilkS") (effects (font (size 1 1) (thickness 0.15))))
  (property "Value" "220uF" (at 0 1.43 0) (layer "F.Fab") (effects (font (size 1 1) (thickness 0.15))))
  (fp_line (start -0.14058 0.51) (end 0.14058 0.51) (stroke (width 0.12) (type solid)) (layer "F.SilkS"))
  (fp_line (start -0.14058 -0.51) (end 0.14058 -0.51) (stroke (width 0.12) (type solid)) (layer "F.SilkS"))
  (pad "1" smd roundrect (at -0.775 0 180) (size 0.9 0.95) (layers "F.Cu" "F.Mask" "F.Paste") (roundrect_rratio 0.25) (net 4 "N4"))
  (pad "2" smd roundrect (at 0.775 0 180) (size 0.9 0.95) (layers "F.Cu" "F.Mask" "F.Paste") (roundrect_rratio 0.25) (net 5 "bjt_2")))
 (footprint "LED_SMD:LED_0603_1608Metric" (layer "F.Cu") (at 126.6 81.8 180)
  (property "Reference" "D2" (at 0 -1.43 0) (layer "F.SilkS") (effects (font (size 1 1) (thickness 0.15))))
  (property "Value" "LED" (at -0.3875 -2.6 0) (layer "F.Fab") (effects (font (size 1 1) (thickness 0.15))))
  (fp_line (start 0.8 -0.735) (end -1.485 -0.735) (stroke (width 0.12) (type solid)) (layer "F.SilkS"))
  (fp_line (start -1.485 0.735) (end 0.8 0.735) (stroke (width 0.12) (type solid)) (layer "F.SilkS"))
  (fp_line (start -1.485 -0.735) (end -1.485 0.735) (stroke (width 0.12) (type solid)) (layer "F.SilkS"))
  (pad "1" smd roundrect (at -0.7875 0 180) (size 0.875 0.95) (layers "F.Cu" "F.Mask" "F.Paste") (roundrect_rratio 0.25) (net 6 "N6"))
  (pad "2" smd roundrect (at 0.7875 0 180) (size 0.875 0.95) (layers "F.Cu" "F.Mask" "F.Paste") (roundrect_rratio 0.25) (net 2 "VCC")))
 (gr_arc (start 119.25 69.6) (mid 120.055456 67.655456) (end 122 66.85) (stroke (width 0.05) (type default)) (layer "Edge.Cuts"))
 (gr_line (start 140.75 69.6) (end 140.757263 85.4) (stroke (width 0.05) (type default)) (layer "Edge.Cuts"))
 (gr_line (start 119.25 69.6) (end 119.25 85.4) (stroke (width 0.05) (type default)) (layer "Edge.Cuts"))
 (gr_line (start 122 88.15) (end 138.2 88.15) (stroke (width 0.05) (type default)) (layer "Edge.Cuts"))
 (gr_arc (start 138 66.85) (mid 139.944544 67.655456) (end 140.75 69.6) (stroke (width 0.05) (type default)) (layer "Edge.Cuts"))
 (gr_arc (start 122 88.15) (mid 120.055456 87.344544) (end 119.25 85.4) (stroke (width 0.05) (type default)) (layer "Edge.Cuts"))
 (gr_line (start 122 66.85) (end 138 66.85) (stroke (width 0.05) (type default)) (layer "Edge.Cuts"))
 (gr_arc (start 140.757263 85.4) (mid 140.019152 87.277638) (end 138.2 88.15) (stroke (width 0.05) (type default)) (layer "Edge.Cuts"))
 (segment (start 133.3875 80.6625) (end 133.4 80.65) (width 0.2) (layer "F.Cu") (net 4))
 (segment (start 135.1375 75.4) (end 132.4 75.4) (width 0.2) (layer "F.Cu") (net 4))
 (segment (start 133.4 78.6) (end 134.243322 78.6) (width 0.2) (layer "F.Cu") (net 4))
 (segment (start 134.243322 78.6) (end 134.443322 78.4) (width 0.2) (layer "F.Cu") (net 4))
 (segment (start 133.3875 81.8) (end 133.3875 80.6625) (width 0.2) (layer "F.Cu") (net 4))
 (segment (start 132.4 75.4) (end 131.2 74.2) (width 0.2) (layer "F.Cu") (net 4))
 (segment (start 134.443322 76.094178) (end 134.443322 78.4) (width 0.2) (layer "F.Cu") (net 4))
 (segment (start 135.1375 75.4) (end 134.443322 76.094178) (width 0.2) (layer "F.Cu") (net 4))
 (via (at 133.4 78.6) (size 0.6) (drill 0.3) (layers "F.Cu" "B.Cu") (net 4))
 (via (at 133.4 80.65) (size 0.6) (drill 0.3) (layers "F.Cu" "B.Cu") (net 4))
 (segment (start 133.4 80.65) (end 133.4 78.6) (width 0.2) (layer "B.Cu") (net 4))
 (segment (start 128.4 80.075) (end 131.375 80.075) (width 0.2) (layer "F.Cu") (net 2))
 (segment (start 125.8125 80.2875) (end 125.6 80.075) (width 0.2) (layer "F.Cu") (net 2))
 (segment (start 126.1875 81.425) (end 125.8125 81.8) (width 0.2) (layer "F.Cu") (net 2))
 (segment (start 125.6 80.075) (end 128.4 80.075) (width 0.2) (layer "F.Cu") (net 2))
 (segment (start 131.8125 81.8) (end 131.8125 80.4625) (width 0.2) (layer "F.Cu") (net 2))
 (segment (start 131.8125 80.4625) (end 131.4 80.05) (width 0.2) (layer "F.Cu") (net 2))
 (segment (start 134.443322 80.05) (end 136.09 80.05) (width 0.2) (layer "F.Cu") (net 2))
 (segment (start 131.375 80.075) (end 131.4 80.05) (width 0.2) (layer "F.Cu") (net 2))
 (segment (start 131.4 80.05) (end 134.443322 80.05) (width 0.2) (layer "F.Cu") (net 2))
 (segment (start 136.09 80.05) (end 138.2 77.94) (width 0.2) (layer "F.Cu") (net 2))
 (segment (start 125.8125 81.8) (end 125.8125 80.2875) (width 0.2) (layer "F.Cu") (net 2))
 (segment (start 129.65 74.2) (end 127.420532 74.2) (width 0.2) (layer "F.Cu") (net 5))
 (segment (start 125.725 75.895532) (end 125.725 76.35) (width 0.2) (layer "F.Cu") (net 5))
 (segment (start 125.6 76.475) (end 125.725 76.35) (width 0.2) (layer "F.Cu") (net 5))
 (segment (start 127.420532 74.2) (end 125.725 75.895532) (width 0.2) (layer "F.Cu") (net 5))
 (segment (start 125.6 78.425) (end 125.6 76.475) (width 0.2) (layer "F.Cu") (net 5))
 (segment (start 131.4 78.4) (end 131.4 76.225) (width 0.2) (layer "F.Cu") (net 3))
 (segment (start 131.175 76) (end 132.9125 76) (width 0.2) (layer "F.Cu") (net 3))
 (segment (start 131.4 76.225) (end 131.175 76) (width 0.2) (layer "F.Cu") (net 3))
 (segment (start 132.9125 76) (end 133.2625 76.35) (width 0.2) (layer "F.Cu") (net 3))
 (segment (start 128.4 76.2) (end 127.6 75.4) (width 0.2) (layer "F.Cu") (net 6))
 (segment (start 129.025 75.4) (end 129.625 76) (width 0.2) (layer "F.Cu") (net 6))
 (segment (start 128.4 78.425) (end 128.4 76.2) (width 0.2) (layer "F.Cu") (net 6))
 (segment (start 127.3875 80.6875) (end 127.4 80.675) (width 0.2) (layer "F.Cu") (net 6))
 (segment (start 127.6 75.4) (end 129.025 75.4) (width 0.2) (layer "F.Cu") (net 6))
 (segment (start 127.4 78.6) (end 128.225 78.6) (width 0.2) (layer "F.Cu") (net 6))
 (segment (start 127.3875 81.8) (end 127.3875 80.6875) (width 0.2) (layer "F.Cu") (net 6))
 (segment (start 128.225 78.6) (end 128.4 78.425) (width 0.2) (layer "F.Cu") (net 6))
 (via (at 127.4 78.6) (size 0.6) (drill 0.3) (layers "F.Cu" "B.Cu") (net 6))
 (via (at 127.4 80.675) (size 0.6) (drill 0.3) (layers "F.Cu" "B.Cu") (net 6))
 (segment (start 127.4 80.675) (end 127.4 78.6) (width 0.2) (layer "B.Cu") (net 6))
 (segment (start 125.725 74.45) (end 122 70.725) (width 0.2) (layer "F.Cu") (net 1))
 (segment (start 137.25 74.45) (end 138.2 75.4) (width 0.2) (layer "F.Cu") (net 1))
 (segment (start 133.2625 74.45) (end 137.25 74.45) (width 0.2) (layer "F.Cu") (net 1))
 (segment (start 122 70.725) (end 122 69.6) (width 0.2) (layer "F.Cu") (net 1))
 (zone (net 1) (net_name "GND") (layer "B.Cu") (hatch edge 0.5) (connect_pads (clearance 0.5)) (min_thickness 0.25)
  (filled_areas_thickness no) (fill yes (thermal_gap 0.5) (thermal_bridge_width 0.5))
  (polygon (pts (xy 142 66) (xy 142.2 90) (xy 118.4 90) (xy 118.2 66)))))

